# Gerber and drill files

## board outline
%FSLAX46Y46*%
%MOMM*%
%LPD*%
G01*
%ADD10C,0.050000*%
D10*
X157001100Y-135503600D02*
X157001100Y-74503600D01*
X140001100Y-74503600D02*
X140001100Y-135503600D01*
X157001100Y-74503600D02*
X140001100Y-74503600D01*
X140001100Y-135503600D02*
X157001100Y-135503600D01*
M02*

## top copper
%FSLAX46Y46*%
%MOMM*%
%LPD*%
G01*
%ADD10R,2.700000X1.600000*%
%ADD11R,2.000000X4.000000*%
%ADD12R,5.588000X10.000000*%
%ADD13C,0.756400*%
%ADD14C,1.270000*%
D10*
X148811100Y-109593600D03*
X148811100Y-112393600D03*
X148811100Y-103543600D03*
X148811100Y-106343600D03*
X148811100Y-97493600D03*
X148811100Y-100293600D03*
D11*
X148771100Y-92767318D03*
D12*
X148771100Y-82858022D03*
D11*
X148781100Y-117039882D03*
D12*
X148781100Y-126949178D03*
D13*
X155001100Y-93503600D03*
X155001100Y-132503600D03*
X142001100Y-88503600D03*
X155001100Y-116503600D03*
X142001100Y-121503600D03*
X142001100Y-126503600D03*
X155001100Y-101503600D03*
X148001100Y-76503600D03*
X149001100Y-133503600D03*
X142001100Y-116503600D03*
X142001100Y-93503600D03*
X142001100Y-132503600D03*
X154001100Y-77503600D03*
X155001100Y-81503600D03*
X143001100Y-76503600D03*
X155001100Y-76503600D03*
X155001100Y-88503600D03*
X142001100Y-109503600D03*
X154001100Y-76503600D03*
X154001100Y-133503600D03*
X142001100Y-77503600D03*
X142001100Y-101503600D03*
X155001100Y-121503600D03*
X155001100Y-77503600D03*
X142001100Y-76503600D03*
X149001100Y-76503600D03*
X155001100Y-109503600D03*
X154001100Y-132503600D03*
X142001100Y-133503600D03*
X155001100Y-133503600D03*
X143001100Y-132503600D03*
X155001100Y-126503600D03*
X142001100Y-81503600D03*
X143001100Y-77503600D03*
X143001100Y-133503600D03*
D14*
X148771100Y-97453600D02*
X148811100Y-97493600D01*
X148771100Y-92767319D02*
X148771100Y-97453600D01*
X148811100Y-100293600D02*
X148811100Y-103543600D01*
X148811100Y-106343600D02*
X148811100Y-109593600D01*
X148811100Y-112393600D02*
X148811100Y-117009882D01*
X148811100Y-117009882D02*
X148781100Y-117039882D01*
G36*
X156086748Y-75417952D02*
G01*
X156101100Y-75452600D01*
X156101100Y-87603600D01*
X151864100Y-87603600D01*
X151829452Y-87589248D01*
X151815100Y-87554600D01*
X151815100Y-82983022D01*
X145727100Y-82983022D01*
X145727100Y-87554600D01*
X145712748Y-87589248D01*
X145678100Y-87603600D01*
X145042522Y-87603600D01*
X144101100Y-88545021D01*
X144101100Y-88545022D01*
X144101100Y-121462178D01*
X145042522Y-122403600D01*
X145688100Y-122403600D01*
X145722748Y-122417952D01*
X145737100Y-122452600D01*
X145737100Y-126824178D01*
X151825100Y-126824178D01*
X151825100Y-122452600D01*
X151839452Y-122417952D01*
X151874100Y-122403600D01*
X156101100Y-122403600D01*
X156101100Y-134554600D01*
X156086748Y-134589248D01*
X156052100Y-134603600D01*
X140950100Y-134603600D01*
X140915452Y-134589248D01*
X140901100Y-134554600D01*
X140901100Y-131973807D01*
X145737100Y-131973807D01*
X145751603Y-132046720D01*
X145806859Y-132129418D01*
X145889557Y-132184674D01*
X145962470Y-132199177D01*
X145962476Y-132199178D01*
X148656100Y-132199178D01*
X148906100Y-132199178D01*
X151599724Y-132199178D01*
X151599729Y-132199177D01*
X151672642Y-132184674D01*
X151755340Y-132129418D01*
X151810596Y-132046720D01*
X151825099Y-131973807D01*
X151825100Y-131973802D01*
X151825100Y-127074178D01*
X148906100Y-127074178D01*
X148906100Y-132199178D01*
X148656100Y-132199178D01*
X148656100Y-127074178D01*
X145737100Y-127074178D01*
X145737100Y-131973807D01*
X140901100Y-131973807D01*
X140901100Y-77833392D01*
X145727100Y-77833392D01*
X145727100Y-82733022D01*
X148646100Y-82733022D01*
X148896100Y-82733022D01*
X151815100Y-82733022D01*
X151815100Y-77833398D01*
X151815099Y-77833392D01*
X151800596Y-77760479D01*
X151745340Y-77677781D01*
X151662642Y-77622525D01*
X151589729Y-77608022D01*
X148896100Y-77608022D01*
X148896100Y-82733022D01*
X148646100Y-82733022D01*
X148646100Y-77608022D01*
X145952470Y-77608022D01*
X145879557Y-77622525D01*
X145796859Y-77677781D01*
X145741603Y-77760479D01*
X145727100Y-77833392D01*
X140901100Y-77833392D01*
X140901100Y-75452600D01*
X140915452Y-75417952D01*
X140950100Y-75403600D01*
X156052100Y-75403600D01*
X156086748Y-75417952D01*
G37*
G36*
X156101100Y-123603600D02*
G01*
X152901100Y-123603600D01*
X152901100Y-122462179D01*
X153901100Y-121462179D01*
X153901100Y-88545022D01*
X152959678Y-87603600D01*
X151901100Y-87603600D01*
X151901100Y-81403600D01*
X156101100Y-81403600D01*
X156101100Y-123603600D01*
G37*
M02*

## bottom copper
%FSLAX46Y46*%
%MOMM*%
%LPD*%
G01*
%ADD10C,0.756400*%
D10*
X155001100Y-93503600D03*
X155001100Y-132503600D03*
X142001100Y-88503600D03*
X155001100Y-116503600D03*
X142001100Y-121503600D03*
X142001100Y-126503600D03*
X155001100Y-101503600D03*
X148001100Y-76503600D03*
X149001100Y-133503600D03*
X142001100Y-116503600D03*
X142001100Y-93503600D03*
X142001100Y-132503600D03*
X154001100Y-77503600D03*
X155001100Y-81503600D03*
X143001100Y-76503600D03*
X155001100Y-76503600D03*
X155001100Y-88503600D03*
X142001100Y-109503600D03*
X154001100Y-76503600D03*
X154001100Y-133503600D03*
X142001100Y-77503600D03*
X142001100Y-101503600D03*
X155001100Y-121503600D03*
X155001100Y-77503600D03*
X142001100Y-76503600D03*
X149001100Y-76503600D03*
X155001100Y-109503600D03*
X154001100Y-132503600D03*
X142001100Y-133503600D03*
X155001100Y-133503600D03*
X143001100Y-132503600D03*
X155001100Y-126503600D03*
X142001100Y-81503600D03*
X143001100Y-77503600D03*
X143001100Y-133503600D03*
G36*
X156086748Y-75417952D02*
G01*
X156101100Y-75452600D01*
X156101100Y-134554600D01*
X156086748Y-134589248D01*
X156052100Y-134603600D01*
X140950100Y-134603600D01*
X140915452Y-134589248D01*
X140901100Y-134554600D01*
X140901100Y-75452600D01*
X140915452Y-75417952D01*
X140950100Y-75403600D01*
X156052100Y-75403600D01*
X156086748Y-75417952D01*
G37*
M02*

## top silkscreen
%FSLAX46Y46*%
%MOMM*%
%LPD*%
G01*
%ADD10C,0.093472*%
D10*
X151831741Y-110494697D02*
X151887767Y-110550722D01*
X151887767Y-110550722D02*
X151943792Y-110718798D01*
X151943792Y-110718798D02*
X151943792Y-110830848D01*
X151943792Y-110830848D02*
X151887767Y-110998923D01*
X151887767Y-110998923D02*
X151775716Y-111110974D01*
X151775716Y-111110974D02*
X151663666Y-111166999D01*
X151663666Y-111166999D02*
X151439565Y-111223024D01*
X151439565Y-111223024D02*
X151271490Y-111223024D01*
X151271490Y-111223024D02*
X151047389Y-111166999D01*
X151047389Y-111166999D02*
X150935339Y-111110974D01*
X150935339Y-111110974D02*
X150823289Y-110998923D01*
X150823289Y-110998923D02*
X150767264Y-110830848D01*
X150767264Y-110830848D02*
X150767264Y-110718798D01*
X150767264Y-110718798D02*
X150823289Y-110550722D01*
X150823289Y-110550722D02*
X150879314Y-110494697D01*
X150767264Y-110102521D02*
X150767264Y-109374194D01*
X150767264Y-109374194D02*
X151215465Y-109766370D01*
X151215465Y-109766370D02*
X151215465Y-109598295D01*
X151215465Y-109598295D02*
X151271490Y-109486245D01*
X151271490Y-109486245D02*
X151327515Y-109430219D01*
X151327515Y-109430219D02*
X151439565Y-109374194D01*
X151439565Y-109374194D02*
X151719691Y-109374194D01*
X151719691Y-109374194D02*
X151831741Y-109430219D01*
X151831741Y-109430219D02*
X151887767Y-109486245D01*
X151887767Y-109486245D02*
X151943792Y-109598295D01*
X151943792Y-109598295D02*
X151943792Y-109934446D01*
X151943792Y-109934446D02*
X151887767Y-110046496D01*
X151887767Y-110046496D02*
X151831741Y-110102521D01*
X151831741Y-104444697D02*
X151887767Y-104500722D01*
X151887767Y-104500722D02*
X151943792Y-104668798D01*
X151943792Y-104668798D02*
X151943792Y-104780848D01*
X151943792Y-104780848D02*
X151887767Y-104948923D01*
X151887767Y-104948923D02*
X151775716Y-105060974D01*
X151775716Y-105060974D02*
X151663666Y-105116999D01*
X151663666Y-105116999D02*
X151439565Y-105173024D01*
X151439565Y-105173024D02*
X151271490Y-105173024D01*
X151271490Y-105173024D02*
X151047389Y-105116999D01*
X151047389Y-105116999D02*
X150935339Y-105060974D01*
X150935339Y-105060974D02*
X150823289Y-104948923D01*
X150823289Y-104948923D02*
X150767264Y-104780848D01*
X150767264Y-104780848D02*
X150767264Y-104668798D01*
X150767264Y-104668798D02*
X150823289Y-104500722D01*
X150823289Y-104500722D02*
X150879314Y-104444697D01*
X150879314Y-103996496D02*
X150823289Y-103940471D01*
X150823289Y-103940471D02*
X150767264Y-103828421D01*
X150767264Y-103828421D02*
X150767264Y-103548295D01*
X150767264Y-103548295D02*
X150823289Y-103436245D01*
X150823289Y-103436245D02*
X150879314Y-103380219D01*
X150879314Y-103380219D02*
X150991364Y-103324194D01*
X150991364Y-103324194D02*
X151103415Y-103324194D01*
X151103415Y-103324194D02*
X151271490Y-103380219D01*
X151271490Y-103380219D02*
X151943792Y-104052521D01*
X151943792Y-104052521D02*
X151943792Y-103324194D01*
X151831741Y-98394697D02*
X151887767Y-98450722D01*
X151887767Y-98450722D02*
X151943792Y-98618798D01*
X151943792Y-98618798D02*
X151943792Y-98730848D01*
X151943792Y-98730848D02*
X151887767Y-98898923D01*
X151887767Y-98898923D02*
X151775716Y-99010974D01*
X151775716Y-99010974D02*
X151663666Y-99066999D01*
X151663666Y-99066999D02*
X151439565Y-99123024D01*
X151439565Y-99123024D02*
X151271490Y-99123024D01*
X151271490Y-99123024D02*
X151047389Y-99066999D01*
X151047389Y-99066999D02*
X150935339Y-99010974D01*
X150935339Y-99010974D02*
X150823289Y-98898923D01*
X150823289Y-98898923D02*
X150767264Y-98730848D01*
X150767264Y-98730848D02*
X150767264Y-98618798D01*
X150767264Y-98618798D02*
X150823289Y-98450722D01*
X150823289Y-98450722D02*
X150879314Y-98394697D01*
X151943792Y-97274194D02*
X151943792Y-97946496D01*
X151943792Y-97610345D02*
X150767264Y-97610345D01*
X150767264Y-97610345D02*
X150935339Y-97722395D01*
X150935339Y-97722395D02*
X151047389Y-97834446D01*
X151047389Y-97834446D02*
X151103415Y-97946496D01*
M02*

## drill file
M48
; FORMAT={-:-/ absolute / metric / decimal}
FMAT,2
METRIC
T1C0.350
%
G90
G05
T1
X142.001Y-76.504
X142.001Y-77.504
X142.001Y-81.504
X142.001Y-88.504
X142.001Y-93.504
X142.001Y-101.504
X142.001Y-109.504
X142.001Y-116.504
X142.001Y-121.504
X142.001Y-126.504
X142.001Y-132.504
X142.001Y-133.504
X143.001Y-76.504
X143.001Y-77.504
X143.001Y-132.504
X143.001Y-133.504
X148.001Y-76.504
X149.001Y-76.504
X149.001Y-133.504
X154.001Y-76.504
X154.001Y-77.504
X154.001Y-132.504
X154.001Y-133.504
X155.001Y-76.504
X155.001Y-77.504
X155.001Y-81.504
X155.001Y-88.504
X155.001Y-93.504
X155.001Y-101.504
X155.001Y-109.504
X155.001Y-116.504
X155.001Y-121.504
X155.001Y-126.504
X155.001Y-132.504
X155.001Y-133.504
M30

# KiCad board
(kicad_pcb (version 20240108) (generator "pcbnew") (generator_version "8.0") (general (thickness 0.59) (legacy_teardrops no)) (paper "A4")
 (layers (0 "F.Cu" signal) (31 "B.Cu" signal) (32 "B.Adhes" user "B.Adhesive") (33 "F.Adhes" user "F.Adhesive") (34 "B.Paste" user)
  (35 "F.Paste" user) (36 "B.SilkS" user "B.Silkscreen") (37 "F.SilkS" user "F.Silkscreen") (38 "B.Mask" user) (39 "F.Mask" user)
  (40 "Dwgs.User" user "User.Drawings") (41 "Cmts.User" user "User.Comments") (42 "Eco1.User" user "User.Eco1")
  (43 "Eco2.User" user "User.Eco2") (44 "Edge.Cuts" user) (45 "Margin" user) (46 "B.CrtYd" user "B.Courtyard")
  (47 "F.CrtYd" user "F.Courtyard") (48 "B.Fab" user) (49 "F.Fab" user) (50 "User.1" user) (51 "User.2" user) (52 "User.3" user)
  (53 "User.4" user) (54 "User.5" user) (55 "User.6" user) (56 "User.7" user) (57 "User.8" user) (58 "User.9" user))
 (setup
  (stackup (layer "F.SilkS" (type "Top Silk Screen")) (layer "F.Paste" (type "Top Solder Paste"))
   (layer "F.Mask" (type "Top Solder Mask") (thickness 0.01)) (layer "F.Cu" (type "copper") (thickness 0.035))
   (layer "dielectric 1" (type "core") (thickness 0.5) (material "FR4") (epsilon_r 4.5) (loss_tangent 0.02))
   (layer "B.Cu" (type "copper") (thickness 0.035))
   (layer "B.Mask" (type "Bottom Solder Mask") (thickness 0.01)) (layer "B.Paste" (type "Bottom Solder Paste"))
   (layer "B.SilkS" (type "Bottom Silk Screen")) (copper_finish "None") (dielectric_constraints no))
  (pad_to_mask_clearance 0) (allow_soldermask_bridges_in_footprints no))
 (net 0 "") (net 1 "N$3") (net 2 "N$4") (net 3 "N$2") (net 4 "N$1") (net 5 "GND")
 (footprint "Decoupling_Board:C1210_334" (layer "F.Cu") (at 148.8111 110.9936 -90)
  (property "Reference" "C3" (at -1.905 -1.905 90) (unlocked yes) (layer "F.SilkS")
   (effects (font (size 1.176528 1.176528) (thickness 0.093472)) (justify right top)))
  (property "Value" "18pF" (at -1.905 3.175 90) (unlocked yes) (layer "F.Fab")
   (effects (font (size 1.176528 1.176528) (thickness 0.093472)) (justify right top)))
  (pad "1" smd rect (at -1.4 0 270) (size 1.6 2.7) (layers "F.Cu" "F.Paste" "F.Mask") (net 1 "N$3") (solder_mask_margin 0.1016)
   (thermal_bridge_angle 0))
  (pad "2" smd rect (at 1.4 0 270) (size 1.6 2.7) (layers "F.Cu" "F.Paste" "F.Mask") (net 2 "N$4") (solder_mask_margin 0.1016)
   (thermal_bridge_angle 0)))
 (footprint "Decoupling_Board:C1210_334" (layer "F.Cu") (at 148.8111 104.9436 -90)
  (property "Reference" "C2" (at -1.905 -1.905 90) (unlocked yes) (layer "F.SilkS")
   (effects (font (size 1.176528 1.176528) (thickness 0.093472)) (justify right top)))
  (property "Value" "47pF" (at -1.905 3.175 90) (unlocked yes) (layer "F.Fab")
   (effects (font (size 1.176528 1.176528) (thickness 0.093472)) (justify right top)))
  (pad "1" smd rect (at -1.4 0 270) (size 1.6 2.7) (layers "F.Cu" "F.Paste" "F.Mask") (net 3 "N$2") (solder_mask_margin 0.1016)
   (thermal_bridge_angle 0))
  (pad "2" smd rect (at 1.4 0 270) (size 1.6 2.7) (layers "F.Cu" "F.Paste" "F.Mask") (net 1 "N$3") (solder_mask_margin 0.1016)
   (thermal_bridge_angle 0)))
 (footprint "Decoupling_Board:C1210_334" (layer "F.Cu") (at 148.8111 98.8936 -90)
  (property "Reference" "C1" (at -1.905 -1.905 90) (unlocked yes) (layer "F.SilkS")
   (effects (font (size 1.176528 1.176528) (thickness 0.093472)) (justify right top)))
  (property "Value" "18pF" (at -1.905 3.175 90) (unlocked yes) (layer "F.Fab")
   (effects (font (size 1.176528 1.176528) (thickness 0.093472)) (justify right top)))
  (pad "1" smd rect (at -1.4 0 270) (size 1.6 2.7) (layers "F.Cu" "F.Paste" "F.Mask") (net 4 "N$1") (solder_mask_margin 0.1016)
   (thermal_bridge_angle 0))
  (pad "2" smd rect (at 1.4 0 270) (size 1.6 2.7) (layers "F.Cu" "F.Paste" "F.Mask") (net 3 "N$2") (solder_mask_margin 0.1016)
   (thermal_bridge_angle 0)))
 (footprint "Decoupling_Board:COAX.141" (layer "F.Cu") (at 148.7711 89.4036 90)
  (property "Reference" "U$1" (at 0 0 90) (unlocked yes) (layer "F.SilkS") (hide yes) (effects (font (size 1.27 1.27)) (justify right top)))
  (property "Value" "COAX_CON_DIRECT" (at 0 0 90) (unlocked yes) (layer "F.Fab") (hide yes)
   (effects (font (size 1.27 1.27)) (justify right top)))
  (pad "P$1" smd rect (at -3.363718 0 90) (size 4 2) (layers "F.Cu" "F.Paste" "F.Mask") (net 4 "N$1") (solder_mask_margin 0.1016)
   (thermal_bridge_angle 0))
  (pad "P$2" smd rect (at 6.545578 0 90) (size 10 5.588) (layers "F.Cu" "F.Paste" "F.Mask") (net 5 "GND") (solder_mask_margin 0.1016)
   (thermal_bridge_angle 0)))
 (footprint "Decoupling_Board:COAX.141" (layer "F.Cu") (at 148.7811 120.4036 -90)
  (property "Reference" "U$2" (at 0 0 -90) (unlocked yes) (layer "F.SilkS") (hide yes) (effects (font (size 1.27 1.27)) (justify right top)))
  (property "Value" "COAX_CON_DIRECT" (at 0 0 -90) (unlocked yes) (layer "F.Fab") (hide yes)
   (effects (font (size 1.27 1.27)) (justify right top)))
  (pad "P$1" smd rect (at -3.363718 0 270) (size 4 2) (layers "F.Cu" "F.Paste" "F.Mask") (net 2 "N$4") (solder_mask_margin 0.1016)
   (thermal_bridge_angle 0))
  (pad "P$2" smd rect (at 6.545578 0 270) (size 10 5.588) (layers "F.Cu" "F.Paste" "F.Mask") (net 5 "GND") (solder_mask_margin 0.1016)
   (thermal_bridge_angle 0)))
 (gr_line (start 157.0011 135.5036) (end 157.0011 74.5036) (stroke (width 0.05) (type solid)) (layer "Edge.Cuts"))
 (gr_line (start 140.0011 74.5036) (end 140.0011 135.5036) (stroke (width 0.05) (type solid)) (layer "Edge.Cuts"))
 (gr_line (start 157.0011 74.5036) (end 140.0011 74.5036) (stroke (width 0.05) (type solid)) (layer "Edge.Cuts"))
 (gr_line (start 140.0011 135.5036) (end 157.0011 135.5036) (stroke (width 0.05) (type solid)) (layer "Edge.Cuts"))
 (segment (start 148.7711 97.4536) (end 148.8111 97.4936) (width 1.27) (layer "F.Cu") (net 4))
 (segment (start 148.7711 92.767319) (end 148.7711 97.4536) (width 1.27) (layer "F.Cu") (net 4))
 (segment (start 148.8111 100.2936) (end 148.8111 103.5436) (width 1.27) (layer "F.Cu") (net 3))
 (segment (start 148.8111 106.3436) (end 148.8111 109.5936) (width 1.27) (layer "F.Cu") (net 1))
 (segment (start 148.8111 112.3936) (end 148.8111 117.009882) (width 1.27) (layer "F.Cu") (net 2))
 (segment (start 148.8111 117.009882) (end 148.7811 117.039882) (width 1.27) (layer "F.Cu") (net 2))
 (via (at 155.0011 93.5036) (size 0.7564) (drill 0.35) (layers "F.Cu" "B.Cu") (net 5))
 (via (at 155.0011 132.5036) (size 0.7564) (drill 0.35) (layers "F.Cu" "B.Cu") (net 5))
 (via (at 142.0011 88.5036) (size 0.7564) (drill 0.35) (layers "F.Cu" "B.Cu") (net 5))
 (via (at 155.0011 116.5036) (size 0.7564) (drill 0.35) (layers "F.Cu" "B.Cu") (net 5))
 (via (at 142.0011 121.5036) (size 0.7564) (drill 0.35) (layers "F.Cu" "B.Cu") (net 5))
 (via (at 142.0011 126.5036) (size 0.7564) (drill 0.35) (layers "F.Cu" "B.Cu") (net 5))
 (via (at 155.0011 101.5036) (size 0.7564) (drill 0.35) (layers "F.Cu" "B.Cu") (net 5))
 (via (at 148.0011 76.5036) (size 0.7564) (drill 0.35) (layers "F.Cu" "B.Cu") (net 5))
 (via (at 149.0011 133.5036) (size 0.7564) (drill 0.35) (layers "F.Cu" "B.Cu") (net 5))
 (via (at 142.0011 116.5036) (size 0.7564) (drill 0.35) (layers "F.Cu" "B.Cu") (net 5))
 (via (at 142.0011 93.5036) (size 0.7564) (drill 0.35) (layers "F.Cu" "B.Cu") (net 5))
 (via (at 142.0011 132.5036) (size 0.7564) (drill 0.35) (layers "F.Cu" "B.Cu") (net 5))
 (via (at 154.0011 77.5036) (size 0.7564) (drill 0.35) (layers "F.Cu" "B.Cu") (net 5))
 (via (at 155.0011 81.5036) (size 0.7564) (drill 0.35) (layers "F.Cu" "B.Cu") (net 5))
 (via (at 143.0011 76.5036) (size 0.7564) (drill 0.35) (layers "F.Cu" "B.Cu") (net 5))
 (via (at 155.0011 76.5036) (size 0.7564) (drill 0.35) (layers "F.Cu" "B.Cu") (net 5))
 (via (at 155.0011 88.5036) (size 0.7564) (drill 0.35) (layers "F.Cu" "B.Cu") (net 5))
 (via (at 142.0011 109.5036) (size 0.7564) (drill 0.35) (layers "F.Cu" "B.Cu") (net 5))
 (via (at 154.0011 76.5036) (size 0.7564) (drill 0.35) (layers "F.Cu" "B.Cu") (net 5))
 (via (at 154.0011 133.5036) (size 0.7564) (drill 0.35) (layers "F.Cu" "B.Cu") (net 5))
 (via (at 142.0011 77.5036) (size 0.7564) (drill 0.35) (layers "F.Cu" "B.Cu") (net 5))
 (via (at 142.0011 101.5036) (size 0.7564) (drill 0.35) (layers "F.Cu" "B.Cu") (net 5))
 (via (at 155.0011 121.5036) (size 0.7564) (drill 0.35) (layers "F.Cu" "B.Cu") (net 5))
 (via (at 155.0011 77.5036) (size 0.7564) (drill 0.35) (layers "F.Cu" "B.Cu") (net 5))
 (via (at 142.0011 76.5036) (size 0.7564) (drill 0.35) (layers "F.Cu" "B.Cu") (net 5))
 (via (at 149.0011 76.5036) (size 0.7564) (drill 0.35) (layers "F.Cu" "B.Cu") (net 5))
 (via (at 155.0011 109.5036) (size 0.7564) (drill 0.35) (layers "F.Cu" "B.Cu") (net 5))
 (via (at 154.0011 132.5036) (size 0.7564) (drill 0.35) (layers "F.Cu" "B.Cu") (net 5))
 (via (at 142.0011 133.5036) (size 0.7564) (drill 0.35) (layers "F.Cu" "B.Cu") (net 5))
 (via (at 155.0011 133.5036) (size 0.7564) (drill 0.35) (layers "F.Cu" "B.Cu") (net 5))
 (via (at 143.0011 132.5036) (size 0.7564) (drill 0.35) (layers "F.Cu" "B.Cu") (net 5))
 (via (at 155.0011 126.5036) (size 0.7564) (drill 0.35) (layers "F.Cu" "B.Cu") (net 5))
 (via (at 142.0011 81.5036) (size 0.7564) (drill 0.35) (layers "F.Cu" "B.Cu") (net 5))
 (via (at 143.0011 77.5036) (size 0.7564) (drill 0.35) (layers "F.Cu" "B.Cu") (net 5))
 (via (at 143.0011 133.5036) (size 0.7564) (drill 0.35) (layers "F.Cu" "B.Cu") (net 5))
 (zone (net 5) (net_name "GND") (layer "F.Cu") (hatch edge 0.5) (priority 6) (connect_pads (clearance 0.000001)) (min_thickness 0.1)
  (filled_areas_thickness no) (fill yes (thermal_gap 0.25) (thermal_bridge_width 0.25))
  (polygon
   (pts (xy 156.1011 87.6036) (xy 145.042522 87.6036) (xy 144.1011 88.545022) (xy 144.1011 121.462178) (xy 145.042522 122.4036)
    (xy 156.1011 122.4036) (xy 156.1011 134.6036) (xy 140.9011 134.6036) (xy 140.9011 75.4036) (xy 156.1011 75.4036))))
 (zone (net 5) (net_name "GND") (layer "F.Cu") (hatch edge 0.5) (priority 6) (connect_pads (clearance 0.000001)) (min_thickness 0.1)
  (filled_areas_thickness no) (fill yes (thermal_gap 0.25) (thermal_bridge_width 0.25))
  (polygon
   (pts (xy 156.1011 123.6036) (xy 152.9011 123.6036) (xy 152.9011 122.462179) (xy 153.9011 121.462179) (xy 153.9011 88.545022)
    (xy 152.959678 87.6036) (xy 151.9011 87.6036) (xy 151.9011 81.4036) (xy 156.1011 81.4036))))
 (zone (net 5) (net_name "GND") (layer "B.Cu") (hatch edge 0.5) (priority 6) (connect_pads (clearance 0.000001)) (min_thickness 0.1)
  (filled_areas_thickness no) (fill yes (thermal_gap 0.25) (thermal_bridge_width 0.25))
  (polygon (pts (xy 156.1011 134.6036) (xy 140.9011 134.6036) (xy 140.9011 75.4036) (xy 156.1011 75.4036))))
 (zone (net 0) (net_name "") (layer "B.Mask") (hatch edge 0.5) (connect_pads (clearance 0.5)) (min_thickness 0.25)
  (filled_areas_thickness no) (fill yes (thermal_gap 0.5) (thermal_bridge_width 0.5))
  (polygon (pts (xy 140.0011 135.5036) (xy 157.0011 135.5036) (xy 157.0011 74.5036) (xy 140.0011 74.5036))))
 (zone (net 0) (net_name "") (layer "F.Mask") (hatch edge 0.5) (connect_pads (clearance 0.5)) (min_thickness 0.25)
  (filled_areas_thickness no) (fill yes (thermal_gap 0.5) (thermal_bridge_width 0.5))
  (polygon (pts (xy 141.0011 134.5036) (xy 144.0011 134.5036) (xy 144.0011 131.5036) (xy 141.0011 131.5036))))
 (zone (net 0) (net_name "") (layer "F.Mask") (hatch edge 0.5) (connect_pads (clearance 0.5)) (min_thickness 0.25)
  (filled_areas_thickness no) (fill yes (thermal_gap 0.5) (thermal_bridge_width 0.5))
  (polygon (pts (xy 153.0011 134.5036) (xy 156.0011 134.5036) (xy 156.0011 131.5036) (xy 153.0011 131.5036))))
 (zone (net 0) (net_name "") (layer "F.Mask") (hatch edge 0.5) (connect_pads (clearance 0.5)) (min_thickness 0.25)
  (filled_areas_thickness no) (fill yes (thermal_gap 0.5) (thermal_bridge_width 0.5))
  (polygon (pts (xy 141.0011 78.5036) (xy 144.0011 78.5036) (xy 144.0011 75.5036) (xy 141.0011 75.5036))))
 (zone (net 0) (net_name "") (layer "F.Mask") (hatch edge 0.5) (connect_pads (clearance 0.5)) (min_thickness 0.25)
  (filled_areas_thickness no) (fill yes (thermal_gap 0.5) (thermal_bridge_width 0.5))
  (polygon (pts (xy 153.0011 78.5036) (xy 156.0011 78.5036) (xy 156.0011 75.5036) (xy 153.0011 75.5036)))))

